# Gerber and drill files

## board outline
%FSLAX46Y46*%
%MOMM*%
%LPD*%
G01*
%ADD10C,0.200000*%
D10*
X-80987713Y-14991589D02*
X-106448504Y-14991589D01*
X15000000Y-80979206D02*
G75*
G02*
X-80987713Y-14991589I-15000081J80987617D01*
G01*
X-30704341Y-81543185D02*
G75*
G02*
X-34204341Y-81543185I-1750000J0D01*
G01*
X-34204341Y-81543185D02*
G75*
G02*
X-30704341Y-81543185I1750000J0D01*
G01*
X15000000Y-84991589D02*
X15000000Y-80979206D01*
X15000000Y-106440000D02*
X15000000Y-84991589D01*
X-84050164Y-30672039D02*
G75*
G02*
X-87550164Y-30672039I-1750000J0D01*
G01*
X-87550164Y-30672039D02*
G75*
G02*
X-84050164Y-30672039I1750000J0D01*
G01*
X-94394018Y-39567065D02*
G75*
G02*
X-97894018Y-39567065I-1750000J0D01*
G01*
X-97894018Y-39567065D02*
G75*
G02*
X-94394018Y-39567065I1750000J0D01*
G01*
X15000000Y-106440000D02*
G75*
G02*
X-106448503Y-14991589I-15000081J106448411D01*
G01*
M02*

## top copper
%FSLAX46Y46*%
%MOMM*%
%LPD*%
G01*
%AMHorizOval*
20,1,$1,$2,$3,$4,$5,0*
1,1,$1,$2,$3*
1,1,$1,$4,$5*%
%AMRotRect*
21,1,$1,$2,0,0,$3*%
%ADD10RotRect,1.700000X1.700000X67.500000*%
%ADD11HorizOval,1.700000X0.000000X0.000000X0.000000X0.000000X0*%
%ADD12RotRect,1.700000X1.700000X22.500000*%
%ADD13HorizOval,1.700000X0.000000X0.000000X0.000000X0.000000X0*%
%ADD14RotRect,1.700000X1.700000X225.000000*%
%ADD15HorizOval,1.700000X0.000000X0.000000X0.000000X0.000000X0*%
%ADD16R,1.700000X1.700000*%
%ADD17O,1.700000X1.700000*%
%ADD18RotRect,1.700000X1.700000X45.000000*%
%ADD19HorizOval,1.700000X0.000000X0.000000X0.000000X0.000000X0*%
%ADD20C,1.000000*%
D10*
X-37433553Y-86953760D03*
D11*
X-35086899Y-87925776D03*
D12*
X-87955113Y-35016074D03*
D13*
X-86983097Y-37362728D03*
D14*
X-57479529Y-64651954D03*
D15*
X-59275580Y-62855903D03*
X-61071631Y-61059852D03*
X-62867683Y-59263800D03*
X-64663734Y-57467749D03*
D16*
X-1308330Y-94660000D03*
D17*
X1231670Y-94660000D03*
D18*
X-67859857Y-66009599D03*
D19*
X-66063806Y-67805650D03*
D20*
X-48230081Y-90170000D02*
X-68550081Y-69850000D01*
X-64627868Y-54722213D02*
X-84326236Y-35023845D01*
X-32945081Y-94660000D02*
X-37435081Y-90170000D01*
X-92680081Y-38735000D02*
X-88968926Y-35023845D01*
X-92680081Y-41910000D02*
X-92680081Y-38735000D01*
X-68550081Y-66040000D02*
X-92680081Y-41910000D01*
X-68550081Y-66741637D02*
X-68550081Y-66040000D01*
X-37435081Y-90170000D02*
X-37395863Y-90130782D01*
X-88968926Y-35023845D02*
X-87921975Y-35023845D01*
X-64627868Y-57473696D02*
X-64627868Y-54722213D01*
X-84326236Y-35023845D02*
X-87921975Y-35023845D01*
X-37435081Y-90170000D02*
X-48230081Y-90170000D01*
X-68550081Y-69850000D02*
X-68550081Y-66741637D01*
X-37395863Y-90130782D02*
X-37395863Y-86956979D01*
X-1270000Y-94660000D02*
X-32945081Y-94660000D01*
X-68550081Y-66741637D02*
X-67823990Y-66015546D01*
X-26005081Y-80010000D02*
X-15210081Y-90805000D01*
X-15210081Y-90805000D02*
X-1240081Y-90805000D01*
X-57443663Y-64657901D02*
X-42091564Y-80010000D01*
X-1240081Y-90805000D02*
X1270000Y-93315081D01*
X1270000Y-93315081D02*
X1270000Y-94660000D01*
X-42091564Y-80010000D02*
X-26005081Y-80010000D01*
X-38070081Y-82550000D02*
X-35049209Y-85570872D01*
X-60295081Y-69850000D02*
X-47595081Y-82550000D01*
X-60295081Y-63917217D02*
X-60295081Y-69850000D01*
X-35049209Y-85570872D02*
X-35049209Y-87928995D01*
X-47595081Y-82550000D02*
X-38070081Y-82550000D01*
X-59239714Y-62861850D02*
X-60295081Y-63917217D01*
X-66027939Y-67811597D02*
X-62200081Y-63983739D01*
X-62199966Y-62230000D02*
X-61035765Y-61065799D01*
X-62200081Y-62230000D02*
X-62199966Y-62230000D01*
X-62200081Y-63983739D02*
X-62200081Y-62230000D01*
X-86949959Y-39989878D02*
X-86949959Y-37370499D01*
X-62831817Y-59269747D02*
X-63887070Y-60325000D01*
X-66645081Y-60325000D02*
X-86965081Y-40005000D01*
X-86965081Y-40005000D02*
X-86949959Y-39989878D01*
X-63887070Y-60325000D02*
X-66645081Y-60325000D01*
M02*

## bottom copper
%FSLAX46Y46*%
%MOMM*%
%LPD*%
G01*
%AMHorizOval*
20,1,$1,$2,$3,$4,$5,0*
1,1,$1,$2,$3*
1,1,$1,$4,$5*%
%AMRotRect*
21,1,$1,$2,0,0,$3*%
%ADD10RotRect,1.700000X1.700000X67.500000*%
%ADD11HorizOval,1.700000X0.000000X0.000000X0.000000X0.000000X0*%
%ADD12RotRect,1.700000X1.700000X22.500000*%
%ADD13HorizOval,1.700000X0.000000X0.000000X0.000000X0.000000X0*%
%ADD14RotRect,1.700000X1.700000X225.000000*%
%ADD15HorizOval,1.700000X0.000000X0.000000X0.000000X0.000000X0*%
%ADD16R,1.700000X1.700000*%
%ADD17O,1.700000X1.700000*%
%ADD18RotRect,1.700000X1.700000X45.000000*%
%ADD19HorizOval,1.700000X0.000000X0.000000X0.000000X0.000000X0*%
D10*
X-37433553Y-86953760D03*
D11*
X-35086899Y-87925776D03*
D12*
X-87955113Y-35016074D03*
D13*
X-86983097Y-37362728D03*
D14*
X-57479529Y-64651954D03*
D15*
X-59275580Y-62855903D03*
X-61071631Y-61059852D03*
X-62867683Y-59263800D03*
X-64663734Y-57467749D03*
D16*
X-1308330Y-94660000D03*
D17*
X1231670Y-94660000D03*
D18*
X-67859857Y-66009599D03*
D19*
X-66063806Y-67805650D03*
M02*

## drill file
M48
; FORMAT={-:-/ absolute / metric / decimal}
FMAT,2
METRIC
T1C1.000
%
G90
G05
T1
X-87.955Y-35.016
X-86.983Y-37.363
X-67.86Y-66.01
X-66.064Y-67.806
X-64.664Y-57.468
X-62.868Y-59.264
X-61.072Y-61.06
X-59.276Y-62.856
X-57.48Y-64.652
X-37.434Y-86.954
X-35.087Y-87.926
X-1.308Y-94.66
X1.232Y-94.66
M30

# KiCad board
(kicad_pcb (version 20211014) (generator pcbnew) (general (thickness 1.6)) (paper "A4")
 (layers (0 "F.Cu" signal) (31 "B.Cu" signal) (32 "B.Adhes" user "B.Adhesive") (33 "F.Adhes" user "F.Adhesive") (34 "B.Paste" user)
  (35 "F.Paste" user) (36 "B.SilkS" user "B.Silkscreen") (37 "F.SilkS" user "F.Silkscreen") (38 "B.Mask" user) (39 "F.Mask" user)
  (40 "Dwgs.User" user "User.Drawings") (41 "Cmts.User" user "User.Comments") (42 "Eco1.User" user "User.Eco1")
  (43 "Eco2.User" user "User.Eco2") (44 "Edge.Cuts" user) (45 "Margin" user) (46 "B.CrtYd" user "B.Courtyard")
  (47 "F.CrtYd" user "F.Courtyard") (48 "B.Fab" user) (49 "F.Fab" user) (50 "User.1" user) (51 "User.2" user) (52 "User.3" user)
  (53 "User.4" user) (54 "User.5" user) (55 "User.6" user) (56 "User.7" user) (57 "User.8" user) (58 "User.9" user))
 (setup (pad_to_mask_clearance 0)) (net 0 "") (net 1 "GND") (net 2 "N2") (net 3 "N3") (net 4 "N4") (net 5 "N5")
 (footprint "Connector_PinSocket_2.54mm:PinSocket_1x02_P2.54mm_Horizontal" (layer "F.Cu") (at -37.433553 86.95376 67.5)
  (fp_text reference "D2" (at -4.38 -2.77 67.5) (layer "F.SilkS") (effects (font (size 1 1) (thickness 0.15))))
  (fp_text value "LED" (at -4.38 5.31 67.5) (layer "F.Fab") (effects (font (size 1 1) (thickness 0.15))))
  (pad "1" thru_hole rect (at 0 0 67.5) (size 1.7 1.7) (drill 1) (layers *.Cu *.Mask) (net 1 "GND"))
  (pad "2" thru_hole oval (at 0 2.54 67.5) (size 1.7 1.7) (drill 1) (layers *.Cu *.Mask) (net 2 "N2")))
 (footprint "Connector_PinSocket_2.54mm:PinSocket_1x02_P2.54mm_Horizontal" (layer "F.Cu") (at -87.955113 35.016074 22.5)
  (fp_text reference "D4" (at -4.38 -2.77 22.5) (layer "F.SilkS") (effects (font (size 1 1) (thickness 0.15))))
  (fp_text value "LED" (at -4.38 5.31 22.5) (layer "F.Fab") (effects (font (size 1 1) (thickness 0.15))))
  (pad "1" thru_hole rect (at 0 0 22.5) (size 1.7 1.7) (drill 1) (layers *.Cu *.Mask) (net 1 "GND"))
  (pad "2" thru_hole oval (at 0 2.54 22.5) (size 1.7 1.7) (drill 1) (layers *.Cu *.Mask) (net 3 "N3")))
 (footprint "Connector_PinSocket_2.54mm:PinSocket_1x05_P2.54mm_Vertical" (layer "F.Cu") (at -57.479529 64.651954 -135)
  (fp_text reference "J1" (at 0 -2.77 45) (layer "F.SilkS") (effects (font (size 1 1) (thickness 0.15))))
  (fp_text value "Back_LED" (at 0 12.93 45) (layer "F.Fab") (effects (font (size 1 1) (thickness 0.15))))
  (pad "1" thru_hole rect (at 0 0 225) (size 1.7 1.7) (drill 1) (layers *.Cu *.Mask) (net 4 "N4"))
  (pad "2" thru_hole oval (at 0 2.54 225) (size 1.7 1.7) (drill 1) (layers *.Cu *.Mask) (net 2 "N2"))
  (pad "3" thru_hole oval (at 0 5.08 225) (size 1.7 1.7) (drill 1) (layers *.Cu *.Mask) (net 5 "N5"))
  (pad "4" thru_hole oval (at 0 7.62 225) (size 1.7 1.7) (drill 1) (layers *.Cu *.Mask) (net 3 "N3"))
  (pad "5" thru_hole oval (at 0 10.16 225) (size 1.7 1.7) (drill 1) (layers *.Cu *.Mask) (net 1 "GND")))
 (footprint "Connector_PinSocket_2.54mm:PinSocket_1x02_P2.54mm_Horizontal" (layer "F.Cu") (at -1.30833 94.66 90)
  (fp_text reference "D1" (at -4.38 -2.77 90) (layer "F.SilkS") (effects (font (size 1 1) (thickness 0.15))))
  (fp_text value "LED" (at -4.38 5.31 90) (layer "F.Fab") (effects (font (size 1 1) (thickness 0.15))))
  (pad "1" thru_hole rect (at 0 0 90) (size 1.7 1.7) (drill 1) (layers *.Cu *.Mask) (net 1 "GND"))
  (pad "2" thru_hole oval (at 0 2.54 90) (size 1.7 1.7) (drill 1) (layers *.Cu *.Mask) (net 4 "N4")))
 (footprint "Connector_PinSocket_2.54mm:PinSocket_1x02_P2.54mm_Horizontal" (layer "F.Cu") (at -67.859857 66.009599 45)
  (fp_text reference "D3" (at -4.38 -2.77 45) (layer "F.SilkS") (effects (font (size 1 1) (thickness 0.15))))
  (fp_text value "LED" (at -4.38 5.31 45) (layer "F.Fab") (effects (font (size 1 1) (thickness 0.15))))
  (pad "1" thru_hole rect (at 0 0 45) (size 1.7 1.7) (drill 1) (layers *.Cu *.Mask) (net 1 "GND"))
  (pad "2" thru_hole oval (at 0 2.54 45) (size 1.7 1.7) (drill 1) (layers *.Cu *.Mask) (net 5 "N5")))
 (gr_line (start -80.987713 14.991589) (end -106.448504 14.991589) (layer "Edge.Cuts") (width 0.2))
 (gr_arc (start 15 80.979206) (mid -46.660349 67.865118) (end -80.987713 14.991589) (layer "Edge.Cuts") (width 0.2))
 (gr_circle (center -32.454341 81.543185) (end -30.704341 81.543185) (layer "Edge.Cuts") (width 0.2) (fill none))
 (gr_line (start 15 84.991589) (end 15 80.979206) (layer "Edge.Cuts") (width 0.2))
 (gr_line (start 15 106.44) (end 15 84.991589) (layer "Edge.Cuts") (width 0.2))
 (gr_circle (center -85.800164 30.672039) (end -84.050164 30.672039) (layer "Edge.Cuts") (width 0.2) (fill none))
 (gr_circle (center -96.144018 39.567065) (end -94.394018 39.567065) (layer "Edge.Cuts") (width 0.2) (fill none))
 (gr_arc (start 15 106.44) (mid -64.663848 85.868617) (end -106.448504 14.991589) (layer "Edge.Cuts") (width 0.2))
 (segment (start -48.230081 90.17) (end -68.550081 69.85) (width 1) (layer "F.Cu") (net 1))
 (segment (start -64.627868 54.722213) (end -84.326236 35.023845) (width 1) (layer "F.Cu") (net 1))
 (segment (start -32.945081 94.66) (end -37.435081 90.17) (width 1) (layer "F.Cu") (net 1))
 (segment (start -92.680081 38.735) (end -88.968926 35.023845) (width 1) (layer "F.Cu") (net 1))
 (segment (start -92.680081 41.91) (end -92.680081 38.735) (width 1) (layer "F.Cu") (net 1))
 (segment (start -68.550081 66.04) (end -92.680081 41.91) (width 1) (layer "F.Cu") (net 1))
 (segment (start -68.550081 66.741637) (end -68.550081 66.04) (width 1) (layer "F.Cu") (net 1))
 (segment (start -37.435081 90.17) (end -37.395863 90.130782) (width 1) (layer "F.Cu") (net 1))
 (segment (start -88.968926 35.023845) (end -87.921975 35.023845) (width 1) (layer "F.Cu") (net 1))
 (segment (start -64.627868 57.473696) (end -64.627868 54.722213) (width 1) (layer "F.Cu") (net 1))
 (segment (start -84.326236 35.023845) (end -87.921975 35.023845) (width 1) (layer "F.Cu") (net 1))
 (segment (start -37.435081 90.17) (end -48.230081 90.17) (width 1) (layer "F.Cu") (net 1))
 (segment (start -68.550081 69.85) (end -68.550081 66.741637) (width 1) (layer "F.Cu") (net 1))
 (segment (start -37.395863 90.130782) (end -37.395863 86.956979) (width 1) (layer "F.Cu") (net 1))
 (segment (start -1.27 94.66) (end -32.945081 94.66) (width 1) (layer "F.Cu") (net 1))
 (segment (start -68.550081 66.741637) (end -67.82399 66.015546) (width 1) (layer "F.Cu") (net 1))
 (segment (start -26.005081 80.01) (end -15.210081 90.805) (width 1) (layer "F.Cu") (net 4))
 (segment (start -15.210081 90.805) (end -1.240081 90.805) (width 1) (layer "F.Cu") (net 4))
 (segment (start -57.443663 64.657901) (end -42.091564 80.01) (width 1) (layer "F.Cu") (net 4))
 (segment (start -1.240081 90.805) (end 1.27 93.315081) (width 1) (layer "F.Cu") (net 4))
 (segment (start 1.27 93.315081) (end 1.27 94.66) (width 1) (layer "F.Cu") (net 4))
 (segment (start -42.091564 80.01) (end -26.005081 80.01) (width 1) (layer "F.Cu") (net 4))
 (segment (start -38.070081 82.55) (end -35.049209 85.570872) (width 1) (layer "F.Cu") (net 2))
 (segment (start -60.295081 69.85) (end -47.595081 82.55) (width 1) (layer "F.Cu") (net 2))
 (segment (start -60.295081 63.917217) (end -60.295081 69.85) (width 1) (layer "F.Cu") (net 2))
 (segment (start -35.049209 85.570872) (end -35.049209 87.928995) (width 1) (layer "F.Cu") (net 2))
 (segment (start -47.595081 82.55) (end -38.070081 82.55) (width 1) (layer "F.Cu") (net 2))
 (segment (start -59.239714 62.86185) (end -60.295081 63.917217) (width 1) (layer "F.Cu") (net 2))
 (segment (start -66.027939 67.811597) (end -62.200081 63.983739) (width 1) (layer "F.Cu") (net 5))
 (segment (start -62.199966 62.23) (end -61.035765 61.065799) (width 1) (layer "F.Cu") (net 5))
 (segment (start -62.200081 62.23) (end -62.199966 62.23) (width 1) (layer "F.Cu") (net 5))
 (segment (start -62.200081 63.983739) (end -62.200081 62.23) (width 1) (layer "F.Cu") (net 5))
 (segment (start -86.949959 39.989878) (end -86.949959 37.370499) (width 1) (layer "F.Cu") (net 3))
 (segment (start -62.831817 59.269747) (end -63.88707 60.325) (width 1) (layer "F.Cu") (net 3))
 (segment (start -66.645081 60.325) (end -86.965081 40.005) (width 1) (layer "F.Cu") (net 3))
 (segment (start -86.965081 40.005) (end -86.949959 39.989878) (width 1) (layer "F.Cu") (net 3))
 (segment (start -63.88707 60.325) (end -66.645081 60.325) (width 1) (layer "F.Cu") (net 3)))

